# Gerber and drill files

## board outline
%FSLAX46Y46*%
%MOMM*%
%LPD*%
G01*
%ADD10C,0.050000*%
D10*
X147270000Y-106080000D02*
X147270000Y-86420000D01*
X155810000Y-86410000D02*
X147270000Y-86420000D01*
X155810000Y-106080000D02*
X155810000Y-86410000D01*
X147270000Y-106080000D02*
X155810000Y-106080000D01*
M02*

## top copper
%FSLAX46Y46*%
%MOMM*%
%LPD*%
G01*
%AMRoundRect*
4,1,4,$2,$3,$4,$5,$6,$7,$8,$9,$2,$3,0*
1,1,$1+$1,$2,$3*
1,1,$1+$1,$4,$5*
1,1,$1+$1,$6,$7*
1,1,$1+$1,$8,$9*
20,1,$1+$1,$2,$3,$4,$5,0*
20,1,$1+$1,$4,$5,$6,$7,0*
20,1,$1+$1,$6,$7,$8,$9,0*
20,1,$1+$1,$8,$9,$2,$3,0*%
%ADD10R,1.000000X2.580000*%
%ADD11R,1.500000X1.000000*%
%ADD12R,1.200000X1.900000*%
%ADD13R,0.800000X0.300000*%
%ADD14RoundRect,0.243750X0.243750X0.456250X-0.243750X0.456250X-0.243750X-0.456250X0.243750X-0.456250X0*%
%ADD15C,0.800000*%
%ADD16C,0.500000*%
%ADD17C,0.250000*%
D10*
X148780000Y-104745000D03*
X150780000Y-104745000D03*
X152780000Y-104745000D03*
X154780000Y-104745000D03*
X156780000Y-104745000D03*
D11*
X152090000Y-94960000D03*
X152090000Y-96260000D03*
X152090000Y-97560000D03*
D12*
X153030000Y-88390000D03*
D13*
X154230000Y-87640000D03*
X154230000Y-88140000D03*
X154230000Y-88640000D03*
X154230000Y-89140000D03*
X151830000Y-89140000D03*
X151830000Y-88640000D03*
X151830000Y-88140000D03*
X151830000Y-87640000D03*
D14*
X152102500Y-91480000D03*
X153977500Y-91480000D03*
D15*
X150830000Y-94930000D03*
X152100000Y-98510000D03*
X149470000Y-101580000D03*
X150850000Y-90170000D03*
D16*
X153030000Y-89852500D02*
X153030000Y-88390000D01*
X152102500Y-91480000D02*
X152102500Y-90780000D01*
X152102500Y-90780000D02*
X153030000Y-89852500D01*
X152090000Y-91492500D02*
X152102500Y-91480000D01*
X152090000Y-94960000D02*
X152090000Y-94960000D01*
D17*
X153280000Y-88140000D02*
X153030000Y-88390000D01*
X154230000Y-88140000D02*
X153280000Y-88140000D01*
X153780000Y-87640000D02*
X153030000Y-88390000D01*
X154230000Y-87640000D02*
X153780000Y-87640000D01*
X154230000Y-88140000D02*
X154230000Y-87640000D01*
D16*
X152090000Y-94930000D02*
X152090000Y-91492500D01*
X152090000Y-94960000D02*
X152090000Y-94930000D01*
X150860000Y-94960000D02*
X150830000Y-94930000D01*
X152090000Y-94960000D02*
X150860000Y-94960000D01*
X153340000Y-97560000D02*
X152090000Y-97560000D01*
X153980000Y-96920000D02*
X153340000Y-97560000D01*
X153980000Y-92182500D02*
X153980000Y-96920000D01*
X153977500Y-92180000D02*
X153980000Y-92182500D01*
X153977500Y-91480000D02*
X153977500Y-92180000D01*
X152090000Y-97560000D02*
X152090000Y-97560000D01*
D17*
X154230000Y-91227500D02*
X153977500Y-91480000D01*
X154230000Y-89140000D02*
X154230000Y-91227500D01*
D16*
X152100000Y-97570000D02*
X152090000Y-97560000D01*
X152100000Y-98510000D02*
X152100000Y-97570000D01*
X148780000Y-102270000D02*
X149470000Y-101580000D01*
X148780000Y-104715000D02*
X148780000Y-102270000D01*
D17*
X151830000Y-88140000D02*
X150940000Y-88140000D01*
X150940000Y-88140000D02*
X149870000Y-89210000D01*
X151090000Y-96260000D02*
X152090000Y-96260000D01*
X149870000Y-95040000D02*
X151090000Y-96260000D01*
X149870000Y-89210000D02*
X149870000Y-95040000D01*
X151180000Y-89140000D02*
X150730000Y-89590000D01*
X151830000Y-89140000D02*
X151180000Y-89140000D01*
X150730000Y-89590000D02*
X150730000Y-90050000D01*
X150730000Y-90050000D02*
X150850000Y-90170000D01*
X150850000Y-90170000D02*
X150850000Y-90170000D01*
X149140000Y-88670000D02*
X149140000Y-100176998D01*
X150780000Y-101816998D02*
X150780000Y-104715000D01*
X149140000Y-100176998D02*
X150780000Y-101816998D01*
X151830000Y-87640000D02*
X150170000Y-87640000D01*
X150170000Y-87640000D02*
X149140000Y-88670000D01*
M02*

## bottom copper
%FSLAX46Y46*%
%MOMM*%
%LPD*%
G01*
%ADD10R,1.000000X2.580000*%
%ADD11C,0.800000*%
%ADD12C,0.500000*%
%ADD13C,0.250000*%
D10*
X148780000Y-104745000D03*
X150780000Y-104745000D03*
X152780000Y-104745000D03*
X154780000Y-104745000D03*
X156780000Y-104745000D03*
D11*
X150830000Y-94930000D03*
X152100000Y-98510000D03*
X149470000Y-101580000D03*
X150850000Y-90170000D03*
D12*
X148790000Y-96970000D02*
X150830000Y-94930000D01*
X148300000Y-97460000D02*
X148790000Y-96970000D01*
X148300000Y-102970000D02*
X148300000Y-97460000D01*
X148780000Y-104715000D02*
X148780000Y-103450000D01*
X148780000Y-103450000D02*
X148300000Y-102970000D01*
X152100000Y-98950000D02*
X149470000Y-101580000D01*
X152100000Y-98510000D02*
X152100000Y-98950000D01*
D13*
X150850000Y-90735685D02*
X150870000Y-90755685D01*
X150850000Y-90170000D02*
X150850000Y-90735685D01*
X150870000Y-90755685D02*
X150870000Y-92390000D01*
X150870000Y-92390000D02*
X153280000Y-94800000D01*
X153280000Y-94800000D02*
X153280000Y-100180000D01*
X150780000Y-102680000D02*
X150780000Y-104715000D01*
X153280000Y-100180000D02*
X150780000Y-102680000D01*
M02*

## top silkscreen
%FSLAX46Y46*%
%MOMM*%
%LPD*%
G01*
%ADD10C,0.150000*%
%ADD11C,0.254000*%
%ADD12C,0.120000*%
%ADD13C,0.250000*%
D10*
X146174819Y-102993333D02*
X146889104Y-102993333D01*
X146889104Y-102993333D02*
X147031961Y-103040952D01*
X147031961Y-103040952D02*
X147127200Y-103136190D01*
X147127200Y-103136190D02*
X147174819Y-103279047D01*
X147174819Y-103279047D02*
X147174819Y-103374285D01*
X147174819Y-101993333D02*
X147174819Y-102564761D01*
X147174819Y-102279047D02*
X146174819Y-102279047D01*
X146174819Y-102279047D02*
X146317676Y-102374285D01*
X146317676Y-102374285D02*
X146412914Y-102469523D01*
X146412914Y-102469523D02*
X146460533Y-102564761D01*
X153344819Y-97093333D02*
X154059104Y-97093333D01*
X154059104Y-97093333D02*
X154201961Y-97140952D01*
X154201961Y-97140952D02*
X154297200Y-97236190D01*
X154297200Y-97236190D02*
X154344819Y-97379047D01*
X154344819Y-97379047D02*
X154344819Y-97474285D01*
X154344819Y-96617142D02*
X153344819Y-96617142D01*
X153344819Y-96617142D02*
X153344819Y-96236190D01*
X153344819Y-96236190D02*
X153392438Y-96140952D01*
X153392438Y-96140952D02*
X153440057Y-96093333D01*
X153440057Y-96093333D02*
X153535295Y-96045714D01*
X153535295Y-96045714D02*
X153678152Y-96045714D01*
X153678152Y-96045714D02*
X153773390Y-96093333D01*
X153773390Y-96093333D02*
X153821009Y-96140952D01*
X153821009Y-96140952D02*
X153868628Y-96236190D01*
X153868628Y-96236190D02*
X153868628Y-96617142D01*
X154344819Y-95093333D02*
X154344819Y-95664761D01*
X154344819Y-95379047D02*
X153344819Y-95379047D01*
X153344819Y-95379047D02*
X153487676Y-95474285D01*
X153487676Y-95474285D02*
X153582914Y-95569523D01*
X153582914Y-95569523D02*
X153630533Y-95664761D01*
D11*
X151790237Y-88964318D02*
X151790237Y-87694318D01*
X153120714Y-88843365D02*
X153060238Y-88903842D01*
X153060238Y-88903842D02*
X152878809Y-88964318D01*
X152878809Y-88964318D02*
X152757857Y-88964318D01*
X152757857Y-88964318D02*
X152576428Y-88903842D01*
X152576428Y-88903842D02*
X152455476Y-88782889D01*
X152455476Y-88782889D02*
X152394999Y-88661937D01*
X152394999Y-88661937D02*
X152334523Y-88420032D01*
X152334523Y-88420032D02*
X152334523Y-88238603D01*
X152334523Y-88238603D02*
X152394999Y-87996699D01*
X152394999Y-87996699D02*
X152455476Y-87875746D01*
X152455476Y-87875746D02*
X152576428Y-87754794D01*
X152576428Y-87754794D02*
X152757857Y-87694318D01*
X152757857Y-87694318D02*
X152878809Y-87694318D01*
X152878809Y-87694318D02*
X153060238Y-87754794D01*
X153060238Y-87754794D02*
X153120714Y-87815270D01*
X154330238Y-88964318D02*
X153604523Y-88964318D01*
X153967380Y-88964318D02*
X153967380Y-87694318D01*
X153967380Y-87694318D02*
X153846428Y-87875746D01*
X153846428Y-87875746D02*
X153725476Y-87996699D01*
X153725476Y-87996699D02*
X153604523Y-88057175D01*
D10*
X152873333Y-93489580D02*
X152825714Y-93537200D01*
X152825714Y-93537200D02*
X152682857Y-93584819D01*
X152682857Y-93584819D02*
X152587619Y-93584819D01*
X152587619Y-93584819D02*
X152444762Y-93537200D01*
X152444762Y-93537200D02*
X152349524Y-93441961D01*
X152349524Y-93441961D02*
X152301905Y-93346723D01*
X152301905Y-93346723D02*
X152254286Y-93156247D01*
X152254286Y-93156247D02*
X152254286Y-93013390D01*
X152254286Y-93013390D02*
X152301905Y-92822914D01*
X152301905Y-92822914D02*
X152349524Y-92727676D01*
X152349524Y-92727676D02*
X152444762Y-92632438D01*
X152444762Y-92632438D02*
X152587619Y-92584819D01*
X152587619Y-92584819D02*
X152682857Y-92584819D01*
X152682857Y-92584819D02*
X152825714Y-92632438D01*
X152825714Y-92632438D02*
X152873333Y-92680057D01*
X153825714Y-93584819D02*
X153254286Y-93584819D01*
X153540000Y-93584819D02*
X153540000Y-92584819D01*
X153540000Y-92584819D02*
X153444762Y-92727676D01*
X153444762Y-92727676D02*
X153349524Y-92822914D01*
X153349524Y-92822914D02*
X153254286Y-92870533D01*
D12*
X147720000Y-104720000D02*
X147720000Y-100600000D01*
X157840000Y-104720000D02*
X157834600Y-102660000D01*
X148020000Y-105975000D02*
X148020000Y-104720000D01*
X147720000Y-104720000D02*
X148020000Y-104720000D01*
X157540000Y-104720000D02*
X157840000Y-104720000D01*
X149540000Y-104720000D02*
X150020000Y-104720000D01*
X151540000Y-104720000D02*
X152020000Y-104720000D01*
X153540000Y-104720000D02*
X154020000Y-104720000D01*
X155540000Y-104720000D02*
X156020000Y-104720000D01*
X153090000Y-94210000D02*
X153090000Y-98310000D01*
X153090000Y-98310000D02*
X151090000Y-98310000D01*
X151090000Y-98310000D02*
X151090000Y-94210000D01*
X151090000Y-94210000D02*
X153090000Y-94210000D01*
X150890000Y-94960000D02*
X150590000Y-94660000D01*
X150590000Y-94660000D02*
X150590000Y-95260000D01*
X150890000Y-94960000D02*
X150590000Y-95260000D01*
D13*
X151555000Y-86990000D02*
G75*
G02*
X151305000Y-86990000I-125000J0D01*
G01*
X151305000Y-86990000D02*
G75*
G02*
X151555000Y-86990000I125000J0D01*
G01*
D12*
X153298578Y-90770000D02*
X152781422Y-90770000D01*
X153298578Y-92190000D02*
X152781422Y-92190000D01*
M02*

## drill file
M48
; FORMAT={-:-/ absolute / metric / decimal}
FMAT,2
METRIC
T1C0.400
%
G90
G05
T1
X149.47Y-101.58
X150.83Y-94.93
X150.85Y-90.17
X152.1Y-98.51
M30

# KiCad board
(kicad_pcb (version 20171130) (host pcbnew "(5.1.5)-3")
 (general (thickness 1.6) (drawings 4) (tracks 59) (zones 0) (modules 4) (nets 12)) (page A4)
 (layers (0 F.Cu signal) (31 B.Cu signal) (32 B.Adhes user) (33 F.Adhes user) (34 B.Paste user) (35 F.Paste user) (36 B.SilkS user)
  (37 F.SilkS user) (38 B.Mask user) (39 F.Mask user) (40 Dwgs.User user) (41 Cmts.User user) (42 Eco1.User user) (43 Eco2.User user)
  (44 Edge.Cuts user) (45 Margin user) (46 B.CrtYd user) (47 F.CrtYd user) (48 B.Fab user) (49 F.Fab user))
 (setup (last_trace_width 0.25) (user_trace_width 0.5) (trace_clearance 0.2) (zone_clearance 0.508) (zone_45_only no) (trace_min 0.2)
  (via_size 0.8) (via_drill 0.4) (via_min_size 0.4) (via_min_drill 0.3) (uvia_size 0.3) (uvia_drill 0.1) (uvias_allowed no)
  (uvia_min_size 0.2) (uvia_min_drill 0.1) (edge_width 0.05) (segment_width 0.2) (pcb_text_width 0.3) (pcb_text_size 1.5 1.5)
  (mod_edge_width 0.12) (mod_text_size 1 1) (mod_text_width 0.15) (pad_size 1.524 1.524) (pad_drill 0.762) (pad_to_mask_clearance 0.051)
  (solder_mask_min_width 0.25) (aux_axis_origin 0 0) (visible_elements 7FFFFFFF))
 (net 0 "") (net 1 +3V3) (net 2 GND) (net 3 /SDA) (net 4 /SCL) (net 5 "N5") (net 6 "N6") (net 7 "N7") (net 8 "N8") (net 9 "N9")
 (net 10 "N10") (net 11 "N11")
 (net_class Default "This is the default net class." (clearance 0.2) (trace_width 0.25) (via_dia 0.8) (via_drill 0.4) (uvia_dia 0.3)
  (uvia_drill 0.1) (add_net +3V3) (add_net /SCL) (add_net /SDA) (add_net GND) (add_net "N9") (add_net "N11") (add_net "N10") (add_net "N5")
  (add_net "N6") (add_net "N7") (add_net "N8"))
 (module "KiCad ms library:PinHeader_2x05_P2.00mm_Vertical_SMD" (layer F.Cu) (at 152.78 102.66 90)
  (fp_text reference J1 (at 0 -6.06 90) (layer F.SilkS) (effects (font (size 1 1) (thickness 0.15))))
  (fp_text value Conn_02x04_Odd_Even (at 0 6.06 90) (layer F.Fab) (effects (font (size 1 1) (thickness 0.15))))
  (fp_line (start -2.06 -5.06) (end 2.06 -5.06) (layer F.SilkS) (width 0.12))
  (fp_line (start -2.06 5.06) (end 0 5.0546) (layer F.SilkS) (width 0.12))
  (fp_line (start -3.315 -4.76) (end -2.06 -4.76) (layer F.SilkS) (width 0.12))
  (fp_line (start -2.06 -5.06) (end -2.06 -4.76) (layer F.SilkS) (width 0.12))
  (fp_line (start -2.06 4.76) (end -2.06 5.06) (layer F.SilkS) (width 0.12))
  (fp_line (start -2.06 -3.24) (end -2.06 -2.76) (layer F.SilkS) (width 0.12))
  (fp_line (start -2.06 -1.24) (end -2.06 -0.76) (layer F.SilkS) (width 0.12))
  (fp_line (start -2.06 0.76) (end -2.06 1.24) (layer F.SilkS) (width 0.12))
  (fp_line (start -2.06 2.76) (end -2.06 3.24) (layer F.SilkS) (width 0.12))
  (pad 1 smd rect (at -2.085 -4 90) (size 2.58 1) (layers F.Cu F.Paste F.Mask) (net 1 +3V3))
  (pad 2 smd rect (at -2.085 -4 270) (size 2.58 1) (layers B.Cu B.Paste B.Mask) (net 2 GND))
  (pad 3 smd rect (at -2.085 -2 90) (size 2.58 1) (layers F.Cu F.Paste F.Mask) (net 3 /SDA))
  (pad 4 smd rect (at -2.085 -2 270) (size 2.58 1) (layers B.Cu B.Paste B.Mask) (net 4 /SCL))
  (pad 5 smd rect (at -2.085 0 90) (size 2.58 1) (layers F.Cu F.Paste F.Mask) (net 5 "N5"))
  (pad 6 smd rect (at -2.085 0 270) (size 2.58 1) (layers B.Cu B.Paste B.Mask) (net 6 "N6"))
  (pad 7 smd rect (at -2.085 2 90) (size 2.58 1) (layers F.Cu F.Paste F.Mask) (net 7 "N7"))
  (pad 8 smd rect (at -2.085 2 270) (size 2.58 1) (layers B.Cu B.Paste B.Mask) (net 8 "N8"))
  (pad 9 smd rect (at -2.085 4 90) (size 2.58 1) (layers F.Cu F.Paste F.Mask))
  (pad 10 smd rect (at -2.085 4 270) (size 2.58 1) (layers B.Cu B.Paste B.Mask)))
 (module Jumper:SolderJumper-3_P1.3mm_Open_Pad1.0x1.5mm (layer F.Cu) (at 152.09 96.26 270)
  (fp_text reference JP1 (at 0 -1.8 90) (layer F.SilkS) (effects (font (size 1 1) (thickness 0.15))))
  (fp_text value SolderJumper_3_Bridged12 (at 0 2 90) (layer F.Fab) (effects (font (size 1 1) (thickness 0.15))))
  (fp_line (start -2.05 -1) (end 2.05 -1) (layer F.SilkS) (width 0.12))
  (fp_line (start 2.05 -1) (end 2.05 1) (layer F.SilkS) (width 0.12))
  (fp_line (start 2.05 1) (end -2.05 1) (layer F.SilkS) (width 0.12))
  (fp_line (start -2.05 1) (end -2.05 -1) (layer F.SilkS) (width 0.12))
  (fp_line (start -1.3 1.2) (end -1.6 1.5) (layer F.SilkS) (width 0.12))
  (fp_line (start -1.6 1.5) (end -1 1.5) (layer F.SilkS) (width 0.12))
  (fp_line (start -1.3 1.2) (end -1 1.5) (layer F.SilkS) (width 0.12))
  (pad 1 smd rect (at -1.3 0 270) (size 1 1.5) (layers F.Cu F.Mask) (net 2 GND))
  (pad 2 smd rect (at 0 0 270) (size 1 1.5) (layers F.Cu F.Mask) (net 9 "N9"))
  (pad 3 smd rect (at 1.3 0 270) (size 1 1.5) (layers F.Cu F.Mask) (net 1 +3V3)))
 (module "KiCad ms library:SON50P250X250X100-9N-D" (layer F.Cu) (at 153.03 88.39)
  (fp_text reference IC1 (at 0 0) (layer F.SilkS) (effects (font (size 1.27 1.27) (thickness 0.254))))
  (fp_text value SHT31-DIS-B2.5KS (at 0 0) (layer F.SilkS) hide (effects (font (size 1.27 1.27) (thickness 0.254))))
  (fp_circle (center -1.6 -1.4) (end -1.6 -1.275) (layer F.SilkS) (width 0.25))
  (pad 9 smd rect (at 0 0) (size 1.2 1.9) (layers F.Cu F.Paste F.Mask) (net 2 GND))
  (pad 8 smd rect (at 1.2 -0.75 90) (size 0.3 0.8) (layers F.Cu F.Paste F.Mask) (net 2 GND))
  (pad 7 smd rect (at 1.2 -0.25 90) (size 0.3 0.8) (layers F.Cu F.Paste F.Mask) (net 2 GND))
  (pad 6 smd rect (at 1.2 0.25 90) (size 0.3 0.8) (layers F.Cu F.Paste F.Mask) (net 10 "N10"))
  (pad 5 smd rect (at 1.2 0.75 90) (size 0.3 0.8) (layers F.Cu F.Paste F.Mask) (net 1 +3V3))
  (pad 4 smd rect (at -1.2 0.75 90) (size 0.3 0.8) (layers F.Cu F.Paste F.Mask) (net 4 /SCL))
  (pad 3 smd rect (at -1.2 0.25 90) (size 0.3 0.8) (layers F.Cu F.Paste F.Mask) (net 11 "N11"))
  (pad 2 smd rect (at -1.2 -0.25 90) (size 0.3 0.8) (layers F.Cu F.Paste F.Mask) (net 9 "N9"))
  (pad 1 smd rect (at -1.2 -0.75 90) (size 0.3 0.8) (layers F.Cu F.Paste F.Mask) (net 3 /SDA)))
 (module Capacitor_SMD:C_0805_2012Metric (layer F.Cu) (at 153.04 91.48 180)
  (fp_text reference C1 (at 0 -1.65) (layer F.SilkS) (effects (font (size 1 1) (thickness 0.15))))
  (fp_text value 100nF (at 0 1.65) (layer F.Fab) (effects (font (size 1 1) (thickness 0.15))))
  (fp_line (start -0.258578 0.71) (end 0.258578 0.71) (layer F.SilkS) (width 0.12))
  (fp_line (start -0.258578 -0.71) (end 0.258578 -0.71) (layer F.SilkS) (width 0.12))
  (pad 2 smd roundrect (at 0.9375 0 180) (size 0.975 1.4) (layers F.Cu F.Paste F.Mask) (roundrect_rratio 0.25) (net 2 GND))
  (pad 1 smd roundrect (at -0.9375 0 180) (size 0.975 1.4) (layers F.Cu F.Paste F.Mask) (roundrect_rratio 0.25) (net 1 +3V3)))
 (gr_line (start 147.27 106.08) (end 147.27 86.42) (layer Edge.Cuts) (width 0.05))
 (gr_line (start 155.81 86.41) (end 147.27 86.42) (layer Edge.Cuts) (width 0.05))
 (gr_line (start 155.81 106.08) (end 155.81 86.41) (layer Edge.Cuts) (width 0.05))
 (gr_line (start 147.27 106.08) (end 155.81 106.08) (layer Edge.Cuts) (width 0.05))
 (segment (start 153.03 89.8525) (end 153.03 88.39) (width 0.5) (layer F.Cu) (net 2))
 (segment (start 152.1025 91.48) (end 152.1025 90.78) (width 0.5) (layer F.Cu) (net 2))
 (segment (start 152.1025 90.78) (end 153.03 89.8525) (width 0.5) (layer F.Cu) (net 2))
 (segment (start 152.09 91.4925) (end 152.1025 91.48) (width 0.5) (layer F.Cu) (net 2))
 (segment (start 152.09 94.96) (end 152.09 94.96) (width 0.5) (layer F.Cu) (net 2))
 (segment (start 153.28 88.14) (end 153.03 88.39) (width 0.25) (layer F.Cu) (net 2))
 (segment (start 154.23 88.14) (end 153.28 88.14) (width 0.25) (layer F.Cu) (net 2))
 (segment (start 153.78 87.64) (end 153.03 88.39) (width 0.25) (layer F.Cu) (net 2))
 (segment (start 154.23 87.64) (end 153.78 87.64) (width 0.25) (layer F.Cu) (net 2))
 (segment (start 154.23 88.14) (end 154.23 87.64) (width 0.25) (layer F.Cu) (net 2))
 (segment (start 152.09 94.93) (end 152.09 91.4925) (width 0.5) (layer F.Cu) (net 2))
 (via (at 150.83 94.93) (size 0.8) (drill 0.4) (layers F.Cu B.Cu) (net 2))
 (segment (start 152.09 94.96) (end 152.09 94.93) (width 0.5) (layer F.Cu) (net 2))
 (segment (start 150.86 94.96) (end 150.83 94.93) (width 0.5) (layer F.Cu) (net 2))
 (segment (start 152.09 94.96) (end 150.86 94.96) (width 0.5) (layer F.Cu) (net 2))
 (segment (start 148.79 96.97) (end 150.83 94.93) (width 0.5) (layer B.Cu) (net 2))
 (segment (start 148.3 97.46) (end 148.79 96.97) (width 0.5) (layer B.Cu) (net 2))
 (segment (start 148.3 102.97) (end 148.3 97.46) (width 0.5) (layer B.Cu) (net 2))
 (segment (start 148.78 104.715) (end 148.78 103.45) (width 0.5) (layer B.Cu) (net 2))
 (segment (start 148.78 103.45) (end 148.3 102.97) (width 0.5) (layer B.Cu) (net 2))
 (segment (start 153.34 97.56) (end 152.09 97.56) (width 0.5) (layer F.Cu) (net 1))
 (segment (start 153.98 96.92) (end 153.34 97.56) (width 0.5) (layer F.Cu) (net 1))
 (segment (start 153.98 92.1825) (end 153.98 96.92) (width 0.5) (layer F.Cu) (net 1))
 (segment (start 153.9775 92.18) (end 153.98 92.1825) (width 0.5) (layer F.Cu) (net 1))
 (segment (start 153.9775 91.48) (end 153.9775 92.18) (width 0.5) (layer F.Cu) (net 1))
 (segment (start 152.09 97.56) (end 152.09 97.56) (width 0.5) (layer F.Cu) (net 1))
 (via (at 152.1 98.51) (size 0.8) (drill 0.4) (layers F.Cu B.Cu) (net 1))
 (via (at 149.47 101.58) (size 0.8) (drill 0.4) (layers F.Cu B.Cu) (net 1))
 (segment (start 154.23 91.2275) (end 153.9775 91.48) (width 0.25) (layer F.Cu) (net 1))
 (segment (start 154.23 89.14) (end 154.23 91.2275) (width 0.25) (layer F.Cu) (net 1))
 (segment (start 152.1 97.57) (end 152.09 97.56) (width 0.5) (layer F.Cu) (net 1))
 (segment (start 152.1 98.51) (end 152.1 97.57) (width 0.5) (layer F.Cu) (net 1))
 (segment (start 148.78 102.27) (end 149.47 101.58) (width 0.5) (layer F.Cu) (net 1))
 (segment (start 148.78 104.715) (end 148.78 102.27) (width 0.5) (layer F.Cu) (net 1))
 (segment (start 152.1 98.95) (end 149.47 101.58) (width 0.5) (layer B.Cu) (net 1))
 (segment (start 152.1 98.51) (end 152.1 98.95) (width 0.5) (layer B.Cu) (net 1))
 (segment (start 151.83 88.14) (end 150.94 88.14) (width 0.25) (layer F.Cu) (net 9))
 (segment (start 150.94 88.14) (end 149.87 89.21) (width 0.25) (layer F.Cu) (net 9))
 (segment (start 151.09 96.26) (end 152.09 96.26) (width 0.25) (layer F.Cu) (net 9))
 (segment (start 149.87 95.04) (end 151.09 96.26) (width 0.25) (layer F.Cu) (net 9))
 (segment (start 149.87 89.21) (end 149.87 95.04) (width 0.25) (layer F.Cu) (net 9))
 (segment (start 151.18 89.14) (end 150.73 89.59) (width 0.25) (layer F.Cu) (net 4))
 (segment (start 151.83 89.14) (end 151.18 89.14) (width 0.25) (layer F.Cu) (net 4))
 (segment (start 150.73 89.59) (end 150.73 90.05) (width 0.25) (layer F.Cu) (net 4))
 (segment (start 150.73 90.05) (end 150.85 90.17) (width 0.25) (layer F.Cu) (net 4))
 (segment (start 150.85 90.17) (end 150.85 90.17) (width 0.25) (layer F.Cu) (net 4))
 (via (at 150.85 90.17) (size 0.8) (drill 0.4) (layers F.Cu B.Cu) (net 4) (status 1000000))
 (segment (start 150.85 90.735685) (end 150.87 90.755685) (width 0.25) (layer B.Cu) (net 4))
 (segment (start 150.85 90.17) (end 150.85 90.735685) (width 0.25) (layer B.Cu) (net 4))
 (segment (start 150.87 90.755685) (end 150.87 92.39) (width 0.25) (layer B.Cu) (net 4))
 (segment (start 150.87 92.39) (end 153.28 94.8) (width 0.25) (layer B.Cu) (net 4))
 (segment (start 153.28 94.8) (end 153.28 100.18) (width 0.25) (layer B.Cu) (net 4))
 (segment (start 150.78 102.68) (end 150.78 104.715) (width 0.25) (layer B.Cu) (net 4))
 (segment (start 153.28 100.18) (end 150.78 102.68) (width 0.25) (layer B.Cu) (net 4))
 (segment (start 149.14 88.67) (end 149.14 100.176998) (width 0.25) (layer F.Cu) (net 3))
 (segment (start 150.78 101.816998) (end 150.78 104.715) (width 0.25) (layer F.Cu) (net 3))
 (segment (start 149.14 100.176998) (end 150.78 101.816998) (width 0.25) (layer F.Cu) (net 3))
 (segment (start 151.83 87.64) (end 150.17 87.64) (width 0.25) (layer F.Cu) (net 3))
 (segment (start 150.17 87.64) (end 149.14 88.67) (width 0.25) (layer F.Cu) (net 3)))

